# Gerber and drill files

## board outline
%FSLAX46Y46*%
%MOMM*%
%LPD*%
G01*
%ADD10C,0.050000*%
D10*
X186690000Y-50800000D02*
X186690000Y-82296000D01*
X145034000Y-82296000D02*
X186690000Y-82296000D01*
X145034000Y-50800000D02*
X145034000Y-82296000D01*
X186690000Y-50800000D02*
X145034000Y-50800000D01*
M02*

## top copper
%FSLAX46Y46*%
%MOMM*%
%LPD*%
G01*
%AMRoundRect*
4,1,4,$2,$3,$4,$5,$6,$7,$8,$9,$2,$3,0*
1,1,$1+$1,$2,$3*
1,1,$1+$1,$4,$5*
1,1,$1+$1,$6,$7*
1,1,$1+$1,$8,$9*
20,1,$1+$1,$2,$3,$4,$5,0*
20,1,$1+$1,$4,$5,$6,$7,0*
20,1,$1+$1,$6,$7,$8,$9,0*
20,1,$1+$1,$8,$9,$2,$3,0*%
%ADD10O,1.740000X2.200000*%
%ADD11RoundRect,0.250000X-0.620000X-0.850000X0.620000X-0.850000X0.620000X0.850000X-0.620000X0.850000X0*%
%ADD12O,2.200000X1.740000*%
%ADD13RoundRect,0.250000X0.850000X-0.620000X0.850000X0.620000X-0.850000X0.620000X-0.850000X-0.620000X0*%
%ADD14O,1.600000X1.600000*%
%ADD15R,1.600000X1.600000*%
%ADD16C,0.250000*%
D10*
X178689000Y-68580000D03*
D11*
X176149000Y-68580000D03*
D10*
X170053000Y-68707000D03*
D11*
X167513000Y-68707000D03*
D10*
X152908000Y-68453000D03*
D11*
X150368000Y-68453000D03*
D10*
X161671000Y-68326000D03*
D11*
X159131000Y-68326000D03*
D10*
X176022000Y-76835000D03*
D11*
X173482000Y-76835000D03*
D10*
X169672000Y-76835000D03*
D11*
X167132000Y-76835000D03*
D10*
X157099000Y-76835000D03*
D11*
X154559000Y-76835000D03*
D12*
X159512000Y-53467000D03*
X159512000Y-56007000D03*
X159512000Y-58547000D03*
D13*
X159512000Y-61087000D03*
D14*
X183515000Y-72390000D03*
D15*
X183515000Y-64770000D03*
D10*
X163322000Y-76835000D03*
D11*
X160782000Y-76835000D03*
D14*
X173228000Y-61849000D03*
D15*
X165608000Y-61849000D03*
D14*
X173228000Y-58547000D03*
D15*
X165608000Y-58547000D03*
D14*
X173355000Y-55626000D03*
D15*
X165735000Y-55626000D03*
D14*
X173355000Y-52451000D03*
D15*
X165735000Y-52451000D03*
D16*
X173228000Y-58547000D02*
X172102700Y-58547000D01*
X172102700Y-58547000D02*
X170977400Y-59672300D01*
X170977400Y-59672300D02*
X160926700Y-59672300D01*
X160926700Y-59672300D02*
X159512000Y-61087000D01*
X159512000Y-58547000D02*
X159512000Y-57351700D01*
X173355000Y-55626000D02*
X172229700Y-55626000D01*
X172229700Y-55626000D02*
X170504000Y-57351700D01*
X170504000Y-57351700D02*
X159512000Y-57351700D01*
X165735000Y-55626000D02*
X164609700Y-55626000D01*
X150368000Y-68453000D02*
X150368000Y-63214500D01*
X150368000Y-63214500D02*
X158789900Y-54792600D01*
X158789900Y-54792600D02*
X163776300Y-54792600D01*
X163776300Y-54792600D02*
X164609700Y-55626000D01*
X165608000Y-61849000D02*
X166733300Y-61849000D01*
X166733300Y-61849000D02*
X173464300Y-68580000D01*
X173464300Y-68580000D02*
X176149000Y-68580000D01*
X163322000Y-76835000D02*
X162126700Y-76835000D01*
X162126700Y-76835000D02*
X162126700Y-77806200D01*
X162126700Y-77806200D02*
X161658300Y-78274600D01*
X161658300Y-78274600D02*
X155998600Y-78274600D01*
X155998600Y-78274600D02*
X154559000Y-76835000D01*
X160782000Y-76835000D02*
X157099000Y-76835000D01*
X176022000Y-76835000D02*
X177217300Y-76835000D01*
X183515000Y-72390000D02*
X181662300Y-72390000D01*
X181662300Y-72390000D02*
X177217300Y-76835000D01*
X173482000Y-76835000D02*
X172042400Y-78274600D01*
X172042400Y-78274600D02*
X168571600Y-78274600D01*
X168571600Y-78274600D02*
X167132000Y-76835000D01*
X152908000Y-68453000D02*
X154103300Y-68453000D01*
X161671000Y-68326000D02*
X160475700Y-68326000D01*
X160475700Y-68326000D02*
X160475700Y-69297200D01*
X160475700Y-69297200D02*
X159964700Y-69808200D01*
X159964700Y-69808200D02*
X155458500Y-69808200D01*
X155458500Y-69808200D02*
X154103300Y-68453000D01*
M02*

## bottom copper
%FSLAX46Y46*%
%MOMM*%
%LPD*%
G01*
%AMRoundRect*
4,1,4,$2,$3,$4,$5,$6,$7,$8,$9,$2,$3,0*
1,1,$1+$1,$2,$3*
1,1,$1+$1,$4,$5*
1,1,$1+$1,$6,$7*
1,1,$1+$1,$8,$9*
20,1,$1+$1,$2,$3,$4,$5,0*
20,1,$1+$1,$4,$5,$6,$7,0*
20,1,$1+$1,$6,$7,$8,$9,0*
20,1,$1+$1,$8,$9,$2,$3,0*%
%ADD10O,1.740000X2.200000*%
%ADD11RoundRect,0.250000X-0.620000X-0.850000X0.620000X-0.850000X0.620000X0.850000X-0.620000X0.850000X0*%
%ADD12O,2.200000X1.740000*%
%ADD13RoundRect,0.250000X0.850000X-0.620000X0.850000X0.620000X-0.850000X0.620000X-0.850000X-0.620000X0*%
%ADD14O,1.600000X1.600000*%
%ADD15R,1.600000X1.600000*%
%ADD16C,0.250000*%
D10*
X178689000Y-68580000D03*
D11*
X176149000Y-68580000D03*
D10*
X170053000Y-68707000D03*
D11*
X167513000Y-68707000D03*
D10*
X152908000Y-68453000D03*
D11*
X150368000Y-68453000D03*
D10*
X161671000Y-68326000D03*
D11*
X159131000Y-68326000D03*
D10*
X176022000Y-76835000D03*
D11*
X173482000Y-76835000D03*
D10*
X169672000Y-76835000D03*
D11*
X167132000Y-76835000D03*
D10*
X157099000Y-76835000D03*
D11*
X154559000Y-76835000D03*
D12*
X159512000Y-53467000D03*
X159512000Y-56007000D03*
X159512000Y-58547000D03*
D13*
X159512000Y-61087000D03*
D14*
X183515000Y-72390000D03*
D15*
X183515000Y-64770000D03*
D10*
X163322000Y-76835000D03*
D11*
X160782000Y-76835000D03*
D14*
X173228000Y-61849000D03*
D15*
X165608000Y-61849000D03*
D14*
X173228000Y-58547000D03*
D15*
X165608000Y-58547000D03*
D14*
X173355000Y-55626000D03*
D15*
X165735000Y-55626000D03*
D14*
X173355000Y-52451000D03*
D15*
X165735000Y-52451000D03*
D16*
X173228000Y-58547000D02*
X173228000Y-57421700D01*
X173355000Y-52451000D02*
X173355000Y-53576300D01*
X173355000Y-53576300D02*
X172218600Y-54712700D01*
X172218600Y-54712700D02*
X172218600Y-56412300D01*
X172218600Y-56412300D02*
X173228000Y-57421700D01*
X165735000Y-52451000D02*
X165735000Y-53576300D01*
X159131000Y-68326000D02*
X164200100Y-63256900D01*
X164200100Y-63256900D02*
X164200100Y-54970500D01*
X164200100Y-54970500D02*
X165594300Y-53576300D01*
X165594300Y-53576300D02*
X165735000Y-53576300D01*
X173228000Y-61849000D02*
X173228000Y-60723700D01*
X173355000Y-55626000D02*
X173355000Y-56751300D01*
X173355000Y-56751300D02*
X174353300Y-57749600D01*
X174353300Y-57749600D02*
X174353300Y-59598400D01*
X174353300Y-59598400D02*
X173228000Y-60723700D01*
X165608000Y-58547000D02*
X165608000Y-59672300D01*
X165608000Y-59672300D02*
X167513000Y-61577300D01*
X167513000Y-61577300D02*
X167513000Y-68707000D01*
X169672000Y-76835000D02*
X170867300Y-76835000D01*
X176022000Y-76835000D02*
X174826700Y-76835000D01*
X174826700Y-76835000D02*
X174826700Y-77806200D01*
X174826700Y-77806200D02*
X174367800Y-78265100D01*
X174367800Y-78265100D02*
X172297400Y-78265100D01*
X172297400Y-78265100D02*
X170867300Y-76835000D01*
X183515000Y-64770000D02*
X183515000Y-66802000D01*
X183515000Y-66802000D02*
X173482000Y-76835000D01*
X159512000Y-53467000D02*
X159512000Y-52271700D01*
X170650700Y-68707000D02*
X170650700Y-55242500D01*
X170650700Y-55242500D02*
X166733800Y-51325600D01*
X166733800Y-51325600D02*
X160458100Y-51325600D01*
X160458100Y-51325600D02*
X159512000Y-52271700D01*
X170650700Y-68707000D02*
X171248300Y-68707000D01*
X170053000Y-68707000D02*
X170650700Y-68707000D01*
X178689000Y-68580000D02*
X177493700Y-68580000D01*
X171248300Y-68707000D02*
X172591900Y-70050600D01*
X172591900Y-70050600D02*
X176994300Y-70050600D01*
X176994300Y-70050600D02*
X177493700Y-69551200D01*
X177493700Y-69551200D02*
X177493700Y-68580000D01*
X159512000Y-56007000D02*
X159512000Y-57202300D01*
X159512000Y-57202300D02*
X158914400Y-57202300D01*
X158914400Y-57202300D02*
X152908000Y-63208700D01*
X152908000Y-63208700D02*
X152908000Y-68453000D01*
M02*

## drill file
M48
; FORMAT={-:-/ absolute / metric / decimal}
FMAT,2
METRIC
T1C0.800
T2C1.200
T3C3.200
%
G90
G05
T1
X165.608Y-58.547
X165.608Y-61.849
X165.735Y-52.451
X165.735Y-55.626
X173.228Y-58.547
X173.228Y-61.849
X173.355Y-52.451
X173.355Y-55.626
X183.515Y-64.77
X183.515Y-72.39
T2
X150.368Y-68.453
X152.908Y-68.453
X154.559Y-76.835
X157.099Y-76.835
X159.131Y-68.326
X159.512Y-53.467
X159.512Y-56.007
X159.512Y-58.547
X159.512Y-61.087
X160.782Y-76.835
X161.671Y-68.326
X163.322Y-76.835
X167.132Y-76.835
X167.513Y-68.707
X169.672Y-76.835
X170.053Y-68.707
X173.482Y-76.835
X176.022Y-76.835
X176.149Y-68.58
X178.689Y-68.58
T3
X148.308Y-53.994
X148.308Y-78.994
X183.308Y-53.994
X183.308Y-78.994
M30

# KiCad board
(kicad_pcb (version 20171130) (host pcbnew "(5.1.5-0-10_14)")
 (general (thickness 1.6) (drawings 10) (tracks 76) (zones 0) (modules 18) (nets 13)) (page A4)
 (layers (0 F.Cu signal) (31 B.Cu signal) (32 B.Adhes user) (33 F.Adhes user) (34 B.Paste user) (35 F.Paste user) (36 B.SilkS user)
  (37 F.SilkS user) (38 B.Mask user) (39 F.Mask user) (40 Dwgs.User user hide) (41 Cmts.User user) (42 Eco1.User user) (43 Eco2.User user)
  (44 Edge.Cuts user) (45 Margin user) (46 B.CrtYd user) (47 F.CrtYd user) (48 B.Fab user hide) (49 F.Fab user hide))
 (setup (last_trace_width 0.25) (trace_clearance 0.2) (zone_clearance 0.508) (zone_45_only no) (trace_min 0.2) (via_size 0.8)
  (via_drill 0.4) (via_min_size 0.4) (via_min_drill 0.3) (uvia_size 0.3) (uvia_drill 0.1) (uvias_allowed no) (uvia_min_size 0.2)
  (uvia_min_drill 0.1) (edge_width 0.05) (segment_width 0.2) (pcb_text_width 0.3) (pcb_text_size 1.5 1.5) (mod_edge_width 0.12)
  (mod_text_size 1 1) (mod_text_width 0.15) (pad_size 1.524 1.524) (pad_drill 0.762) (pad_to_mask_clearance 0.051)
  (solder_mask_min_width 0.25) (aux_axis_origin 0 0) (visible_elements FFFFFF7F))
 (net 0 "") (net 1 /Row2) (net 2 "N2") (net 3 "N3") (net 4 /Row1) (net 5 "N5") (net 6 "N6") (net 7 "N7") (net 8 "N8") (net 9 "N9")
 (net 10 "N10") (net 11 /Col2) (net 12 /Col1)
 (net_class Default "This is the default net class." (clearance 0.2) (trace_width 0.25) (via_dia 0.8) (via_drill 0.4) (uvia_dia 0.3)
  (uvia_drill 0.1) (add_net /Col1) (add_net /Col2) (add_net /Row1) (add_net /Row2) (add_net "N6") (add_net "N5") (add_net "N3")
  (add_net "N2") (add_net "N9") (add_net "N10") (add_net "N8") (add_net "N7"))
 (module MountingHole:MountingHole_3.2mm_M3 (layer F.Cu) (at 183.308 78.994)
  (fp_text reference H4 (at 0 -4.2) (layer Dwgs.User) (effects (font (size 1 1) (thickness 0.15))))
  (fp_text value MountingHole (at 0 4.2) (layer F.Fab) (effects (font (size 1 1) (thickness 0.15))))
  (pad 1 np_thru_hole circle (at 0 0) (size 3.2 3.2) (drill 3.2) (layers *.Cu *.Mask)))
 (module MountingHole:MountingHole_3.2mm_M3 (layer F.Cu) (at 183.308 53.994)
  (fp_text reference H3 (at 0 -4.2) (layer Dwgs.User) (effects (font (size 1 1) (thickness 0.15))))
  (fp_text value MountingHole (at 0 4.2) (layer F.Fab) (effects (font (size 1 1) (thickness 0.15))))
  (pad 1 np_thru_hole circle (at 0 0) (size 3.2 3.2) (drill 3.2) (layers *.Cu *.Mask)))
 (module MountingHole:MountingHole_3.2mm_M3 (layer F.Cu) (at 148.308 53.994)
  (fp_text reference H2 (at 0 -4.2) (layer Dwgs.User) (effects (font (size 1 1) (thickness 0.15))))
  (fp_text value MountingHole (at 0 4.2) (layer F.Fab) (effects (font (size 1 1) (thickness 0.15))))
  (pad 1 np_thru_hole circle (at 0 0) (size 3.2 3.2) (drill 3.2) (layers *.Cu *.Mask)))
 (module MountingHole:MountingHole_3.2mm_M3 (layer F.Cu) (at 148.308 78.994)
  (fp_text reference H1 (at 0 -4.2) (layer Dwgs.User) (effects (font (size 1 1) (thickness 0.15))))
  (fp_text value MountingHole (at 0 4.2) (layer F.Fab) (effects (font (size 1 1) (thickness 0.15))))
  (pad 1 np_thru_hole circle (at 0 0) (size 3.2 3.2) (drill 3.2) (layers *.Cu *.Mask)))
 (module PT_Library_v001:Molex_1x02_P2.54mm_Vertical (layer F.Cu) (at 176.149 68.58)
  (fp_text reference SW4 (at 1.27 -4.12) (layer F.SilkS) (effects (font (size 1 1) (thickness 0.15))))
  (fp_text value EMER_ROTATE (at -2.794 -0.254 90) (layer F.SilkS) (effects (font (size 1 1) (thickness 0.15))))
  (pad 2 thru_hole oval (at 2.54 0) (size 1.74 2.2) (drill 1.2) (layers *.Cu *.Mask) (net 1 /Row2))
  (pad 1 thru_hole roundrect (at 0 0) (size 1.74 2.2) (drill 1.2) (layers *.Cu *.Mask) (roundrect_rratio 0.143678) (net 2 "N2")))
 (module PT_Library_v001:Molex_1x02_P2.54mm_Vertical (layer F.Cu) (at 167.513 68.707)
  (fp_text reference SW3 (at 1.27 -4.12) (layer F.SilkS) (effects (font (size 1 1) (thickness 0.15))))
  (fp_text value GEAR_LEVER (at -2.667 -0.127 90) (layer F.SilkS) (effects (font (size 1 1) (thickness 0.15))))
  (pad 2 thru_hole oval (at 2.54 0) (size 1.74 2.2) (drill 1.2) (layers *.Cu *.Mask) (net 1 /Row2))
  (pad 1 thru_hole roundrect (at 0 0) (size 1.74 2.2) (drill 1.2) (layers *.Cu *.Mask) (roundrect_rratio 0.143678) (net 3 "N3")))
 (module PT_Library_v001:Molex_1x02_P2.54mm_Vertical (layer F.Cu) (at 150.368 68.453)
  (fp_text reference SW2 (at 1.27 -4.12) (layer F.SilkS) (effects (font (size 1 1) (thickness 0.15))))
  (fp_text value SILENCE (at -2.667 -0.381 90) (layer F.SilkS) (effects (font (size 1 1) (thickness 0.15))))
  (pad 2 thru_hole oval (at 2.54 0) (size 1.74 2.2) (drill 1.2) (layers *.Cu *.Mask) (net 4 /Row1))
  (pad 1 thru_hole roundrect (at 0 0) (size 1.74 2.2) (drill 1.2) (layers *.Cu *.Mask) (roundrect_rratio 0.143678) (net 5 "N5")))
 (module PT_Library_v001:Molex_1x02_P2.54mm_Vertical (layer F.Cu) (at 159.131 68.326)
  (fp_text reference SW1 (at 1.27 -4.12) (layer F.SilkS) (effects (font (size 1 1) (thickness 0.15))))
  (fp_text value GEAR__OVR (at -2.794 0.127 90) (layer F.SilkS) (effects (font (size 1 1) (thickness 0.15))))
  (pad 2 thru_hole oval (at 2.54 0) (size 1.74 2.2) (drill 1.2) (layers *.Cu *.Mask) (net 4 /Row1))
  (pad 1 thru_hole roundrect (at 0 0) (size 1.74 2.2) (drill 1.2) (layers *.Cu *.Mask) (roundrect_rratio 0.143678) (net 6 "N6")))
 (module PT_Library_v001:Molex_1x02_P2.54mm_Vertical (layer F.Cu) (at 173.482 76.835)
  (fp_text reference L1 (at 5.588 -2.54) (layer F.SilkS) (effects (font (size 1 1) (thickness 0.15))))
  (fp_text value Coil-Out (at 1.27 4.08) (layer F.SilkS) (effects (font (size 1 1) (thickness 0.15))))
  (pad 2 thru_hole oval (at 2.54 0) (size 1.74 2.2) (drill 1.2) (layers *.Cu *.Mask) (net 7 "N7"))
  (pad 1 thru_hole roundrect (at 0 0) (size 1.74 2.2) (drill 1.2) (layers *.Cu *.Mask) (roundrect_rratio 0.143678) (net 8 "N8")))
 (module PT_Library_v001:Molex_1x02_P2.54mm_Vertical (layer F.Cu) (at 167.132 76.835)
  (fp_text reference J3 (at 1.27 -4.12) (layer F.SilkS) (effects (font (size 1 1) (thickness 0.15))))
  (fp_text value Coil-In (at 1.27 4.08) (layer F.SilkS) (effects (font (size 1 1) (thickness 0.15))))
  (pad 2 thru_hole oval (at 2.54 0) (size 1.74 2.2) (drill 1.2) (layers *.Cu *.Mask) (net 7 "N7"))
  (pad 1 thru_hole roundrect (at 0 0) (size 1.74 2.2) (drill 1.2) (layers *.Cu *.Mask) (roundrect_rratio 0.143678) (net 8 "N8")))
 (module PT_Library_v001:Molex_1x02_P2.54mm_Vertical (layer F.Cu) (at 154.559 76.835)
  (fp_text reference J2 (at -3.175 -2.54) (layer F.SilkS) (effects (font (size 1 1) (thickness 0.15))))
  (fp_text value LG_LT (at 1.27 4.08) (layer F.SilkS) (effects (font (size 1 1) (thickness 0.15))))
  (pad 2 thru_hole oval (at 2.54 0) (size 1.74 2.2) (drill 1.2) (layers *.Cu *.Mask) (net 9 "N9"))
  (pad 1 thru_hole roundrect (at 0 0) (size 1.74 2.2) (drill 1.2) (layers *.Cu *.Mask) (roundrect_rratio 0.143678) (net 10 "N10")))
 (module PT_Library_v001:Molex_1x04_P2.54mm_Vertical (layer F.Cu) (at 159.512 61.087 90)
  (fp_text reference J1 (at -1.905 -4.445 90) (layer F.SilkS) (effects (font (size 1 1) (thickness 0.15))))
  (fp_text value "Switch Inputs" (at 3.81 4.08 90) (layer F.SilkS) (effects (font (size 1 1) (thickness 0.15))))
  (pad 4 thru_hole oval (at 7.62 0 90) (size 1.74 2.2) (drill 1.2) (layers *.Cu *.Mask) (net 1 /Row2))
  (pad 3 thru_hole oval (at 5.08 0 90) (size 1.74 2.2) (drill 1.2) (layers *.Cu *.Mask) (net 4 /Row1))
  (pad 2 thru_hole oval (at 2.54 0 90) (size 1.74 2.2) (drill 1.2) (layers *.Cu *.Mask) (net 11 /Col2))
  (pad 1 thru_hole roundrect (at 0 0 90) (size 1.74 2.2) (drill 1.2) (layers *.Cu *.Mask) (roundrect_rratio 0.143678) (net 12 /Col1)))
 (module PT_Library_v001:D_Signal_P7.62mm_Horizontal (layer F.Cu) (at 183.515 64.77 270)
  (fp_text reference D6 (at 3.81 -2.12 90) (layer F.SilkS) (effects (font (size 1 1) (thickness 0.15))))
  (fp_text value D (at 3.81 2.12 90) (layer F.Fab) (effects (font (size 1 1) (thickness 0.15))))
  (pad 2 thru_hole oval (at 7.62 0 270) (size 1.6 1.6) (drill 0.8) (layers *.Cu *.Mask) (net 7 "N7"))
  (pad 1 thru_hole rect (at 0 0 270) (size 1.6 1.6) (drill 0.8) (layers *.Cu *.Mask) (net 8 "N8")))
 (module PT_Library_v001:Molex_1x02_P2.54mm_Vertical (layer F.Cu) (at 160.782 76.835)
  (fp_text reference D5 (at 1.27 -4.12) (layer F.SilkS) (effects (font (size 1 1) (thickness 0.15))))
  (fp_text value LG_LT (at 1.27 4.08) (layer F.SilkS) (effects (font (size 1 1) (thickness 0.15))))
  (pad 2 thru_hole oval (at 2.54 0) (size 1.74 2.2) (drill 1.2) (layers *.Cu *.Mask) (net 10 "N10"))
  (pad 1 thru_hole roundrect (at 0 0) (size 1.74 2.2) (drill 1.2) (layers *.Cu *.Mask) (roundrect_rratio 0.143678) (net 9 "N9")))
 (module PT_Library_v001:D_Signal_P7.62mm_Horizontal (layer F.Cu) (at 165.608 61.849)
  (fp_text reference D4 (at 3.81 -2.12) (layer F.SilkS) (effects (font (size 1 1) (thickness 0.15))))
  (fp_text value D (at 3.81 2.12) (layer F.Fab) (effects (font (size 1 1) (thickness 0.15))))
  (pad 2 thru_hole oval (at 7.62 0) (size 1.6 1.6) (drill 0.8) (layers *.Cu *.Mask) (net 11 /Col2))
  (pad 1 thru_hole rect (at 0 0) (size 1.6 1.6) (drill 0.8) (layers *.Cu *.Mask) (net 2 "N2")))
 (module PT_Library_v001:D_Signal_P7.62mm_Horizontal (layer F.Cu) (at 165.608 58.547)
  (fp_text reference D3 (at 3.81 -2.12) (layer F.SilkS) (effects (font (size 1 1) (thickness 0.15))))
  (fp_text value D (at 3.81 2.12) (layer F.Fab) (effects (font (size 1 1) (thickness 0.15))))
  (pad 2 thru_hole oval (at 7.62 0) (size 1.6 1.6) (drill 0.8) (layers *.Cu *.Mask) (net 12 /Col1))
  (pad 1 thru_hole rect (at 0 0) (size 1.6 1.6) (drill 0.8) (layers *.Cu *.Mask) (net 3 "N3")))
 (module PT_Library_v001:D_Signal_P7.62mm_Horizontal (layer F.Cu) (at 165.735 55.626)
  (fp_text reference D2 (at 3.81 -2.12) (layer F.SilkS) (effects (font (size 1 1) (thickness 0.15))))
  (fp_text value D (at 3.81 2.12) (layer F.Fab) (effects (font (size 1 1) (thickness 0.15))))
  (pad 2 thru_hole oval (at 7.62 0) (size 1.6 1.6) (drill 0.8) (layers *.Cu *.Mask) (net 11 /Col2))
  (pad 1 thru_hole rect (at 0 0) (size 1.6 1.6) (drill 0.8) (layers *.Cu *.Mask) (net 5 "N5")))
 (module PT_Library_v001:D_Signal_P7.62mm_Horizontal (layer F.Cu) (at 165.735 52.451)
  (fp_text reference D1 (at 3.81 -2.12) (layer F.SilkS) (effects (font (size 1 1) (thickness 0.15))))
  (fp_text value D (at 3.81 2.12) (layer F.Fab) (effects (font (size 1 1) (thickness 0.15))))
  (pad 2 thru_hole oval (at 7.62 0) (size 1.6 1.6) (drill 0.8) (layers *.Cu *.Mask) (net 12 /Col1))
  (pad 1 thru_hole rect (at 0 0) (size 1.6 1.6) (drill 0.8) (layers *.Cu *.Mask) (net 6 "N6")))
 (gr_line (start 186.69 50.8) (end 186.69 82.296) (layer Edge.Cuts) (width 0.05))
 (gr_line (start 145.034 82.296) (end 186.69 82.296) (layer Edge.Cuts) (width 0.05))
 (gr_line (start 145.034 50.8) (end 145.034 82.296) (layer Edge.Cuts) (width 0.05))
 (gr_line (start 186.69 50.8) (end 145.034 50.8) (layer Edge.Cuts) (width 0.05))
 (segment (start 173.228 58.547) (end 173.228 57.4217) (width 0.25) (layer B.Cu) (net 12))
 (segment (start 173.355 52.451) (end 173.355 53.5763) (width 0.25) (layer B.Cu) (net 12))
 (segment (start 173.355 53.5763) (end 172.2186 54.7127) (width 0.25) (layer B.Cu) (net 12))
 (segment (start 172.2186 54.7127) (end 172.2186 56.4123) (width 0.25) (layer B.Cu) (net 12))
 (segment (start 172.2186 56.4123) (end 173.228 57.4217) (width 0.25) (layer B.Cu) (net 12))
 (segment (start 173.228 58.547) (end 172.1027 58.547) (width 0.25) (layer F.Cu) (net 12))
 (segment (start 172.1027 58.547) (end 170.9774 59.6723) (width 0.25) (layer F.Cu) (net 12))
 (segment (start 170.9774 59.6723) (end 160.9267 59.6723) (width 0.25) (layer F.Cu) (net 12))
 (segment (start 160.9267 59.6723) (end 159.512 61.087) (width 0.25) (layer F.Cu) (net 12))
 (segment (start 165.735 52.451) (end 165.735 53.5763) (width 0.25) (layer B.Cu) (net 6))
 (segment (start 159.131 68.326) (end 164.2001 63.2569) (width 0.25) (layer B.Cu) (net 6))
 (segment (start 164.2001 63.2569) (end 164.2001 54.9705) (width 0.25) (layer B.Cu) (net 6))
 (segment (start 164.2001 54.9705) (end 165.5943 53.5763) (width 0.25) (layer B.Cu) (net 6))
 (segment (start 165.5943 53.5763) (end 165.735 53.5763) (width 0.25) (layer B.Cu) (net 6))
 (segment (start 159.512 58.547) (end 159.512 57.3517) (width 0.25) (layer F.Cu) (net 11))
 (segment (start 173.355 55.626) (end 172.2297 55.626) (width 0.25) (layer F.Cu) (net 11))
 (segment (start 172.2297 55.626) (end 170.504 57.3517) (width 0.25) (layer F.Cu) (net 11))
 (segment (start 170.504 57.3517) (end 159.512 57.3517) (width 0.25) (layer F.Cu) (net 11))
 (segment (start 173.228 61.849) (end 173.228 60.7237) (width 0.25) (layer B.Cu) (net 11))
 (segment (start 173.355 55.626) (end 173.355 56.7513) (width 0.25) (layer B.Cu) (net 11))
 (segment (start 173.355 56.7513) (end 174.3533 57.7496) (width 0.25) (layer B.Cu) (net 11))
 (segment (start 174.3533 57.7496) (end 174.3533 59.5984) (width 0.25) (layer B.Cu) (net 11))
 (segment (start 174.3533 59.5984) (end 173.228 60.7237) (width 0.25) (layer B.Cu) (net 11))
 (segment (start 165.735 55.626) (end 164.6097 55.626) (width 0.25) (layer F.Cu) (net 5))
 (segment (start 150.368 68.453) (end 150.368 63.2145) (width 0.25) (layer F.Cu) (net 5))
 (segment (start 150.368 63.2145) (end 158.7899 54.7926) (width 0.25) (layer F.Cu) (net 5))
 (segment (start 158.7899 54.7926) (end 163.7763 54.7926) (width 0.25) (layer F.Cu) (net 5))
 (segment (start 163.7763 54.7926) (end 164.6097 55.626) (width 0.25) (layer F.Cu) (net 5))
 (segment (start 165.608 58.547) (end 165.608 59.6723) (width 0.25) (layer B.Cu) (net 3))
 (segment (start 165.608 59.6723) (end 167.513 61.5773) (width 0.25) (layer B.Cu) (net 3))
 (segment (start 167.513 61.5773) (end 167.513 68.707) (width 0.25) (layer B.Cu) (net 3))
 (segment (start 165.608 61.849) (end 166.7333 61.849) (width 0.25) (layer F.Cu) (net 2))
 (segment (start 166.7333 61.849) (end 173.4643 68.58) (width 0.25) (layer F.Cu) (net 2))
 (segment (start 173.4643 68.58) (end 176.149 68.58) (width 0.25) (layer F.Cu) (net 2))
 (segment (start 163.322 76.835) (end 162.1267 76.835) (width 0.25) (layer F.Cu) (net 10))
 (segment (start 162.1267 76.835) (end 162.1267 77.8062) (width 0.25) (layer F.Cu) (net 10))
 (segment (start 162.1267 77.8062) (end 161.6583 78.2746) (width 0.25) (layer F.Cu) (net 10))
 (segment (start 161.6583 78.2746) (end 155.9986 78.2746) (width 0.25) (layer F.Cu) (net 10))
 (segment (start 155.9986 78.2746) (end 154.559 76.835) (width 0.25) (layer F.Cu) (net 10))
 (segment (start 160.782 76.835) (end 157.099 76.835) (width 0.25) (layer F.Cu) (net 9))
 (segment (start 169.672 76.835) (end 170.8673 76.835) (width 0.25) (layer B.Cu) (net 7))
 (segment (start 176.022 76.835) (end 174.8267 76.835) (width 0.25) (layer B.Cu) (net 7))
 (segment (start 174.8267 76.835) (end 174.8267 77.8062) (width 0.25) (layer B.Cu) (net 7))
 (segment (start 174.8267 77.8062) (end 174.3678 78.2651) (width 0.25) (layer B.Cu) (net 7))
 (segment (start 174.3678 78.2651) (end 172.2974 78.2651) (width 0.25) (layer B.Cu) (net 7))
 (segment (start 172.2974 78.2651) (end 170.8673 76.835) (width 0.25) (layer B.Cu) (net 7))
 (segment (start 176.022 76.835) (end 177.2173 76.835) (width 0.25) (layer F.Cu) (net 7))
 (segment (start 183.515 72.39) (end 181.6623 72.39) (width 0.25) (layer F.Cu) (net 7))
 (segment (start 181.6623 72.39) (end 177.2173 76.835) (width 0.25) (layer F.Cu) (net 7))
 (segment (start 173.482 76.835) (end 172.0424 78.2746) (width 0.25) (layer F.Cu) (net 8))
 (segment (start 172.0424 78.2746) (end 168.5716 78.2746) (width 0.25) (layer F.Cu) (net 8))
 (segment (start 168.5716 78.2746) (end 167.132 76.835) (width 0.25) (layer F.Cu) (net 8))
 (segment (start 183.515 64.77) (end 183.515 66.802) (width 0.25) (layer B.Cu) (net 8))
 (segment (start 183.515 66.802) (end 173.482 76.835) (width 0.25) (layer B.Cu) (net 8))
 (segment (start 159.512 53.467) (end 159.512 52.2717) (width 0.25) (layer B.Cu) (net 1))
 (segment (start 170.6507 68.707) (end 170.6507 55.2425) (width 0.25) (layer B.Cu) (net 1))
 (segment (start 170.6507 55.2425) (end 166.7338 51.3256) (width 0.25) (layer B.Cu) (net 1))
 (segment (start 166.7338 51.3256) (end 160.4581 51.3256) (width 0.25) (layer B.Cu) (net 1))
 (segment (start 160.4581 51.3256) (end 159.512 52.2717) (width 0.25) (layer B.Cu) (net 1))
 (segment (start 170.6507 68.707) (end 171.2483 68.707) (width 0.25) (layer B.Cu) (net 1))
 (segment (start 170.053 68.707) (end 170.6507 68.707) (width 0.25) (layer B.Cu) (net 1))
 (segment (start 178.689 68.58) (end 177.4937 68.58) (width 0.25) (layer B.Cu) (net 1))
 (segment (start 171.2483 68.707) (end 172.5919 70.0506) (width 0.25) (layer B.Cu) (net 1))
 (segment (start 172.5919 70.0506) (end 176.9943 70.0506) (width 0.25) (layer B.Cu) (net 1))
 (segment (start 176.9943 70.0506) (end 177.4937 69.5512) (width 0.25) (layer B.Cu) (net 1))
 (segment (start 177.4937 69.5512) (end 177.4937 68.58) (width 0.25) (layer B.Cu) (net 1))
 (segment (start 152.908 68.453) (end 154.1033 68.453) (width 0.25) (layer F.Cu) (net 4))
 (segment (start 161.671 68.326) (end 160.4757 68.326) (width 0.25) (layer F.Cu) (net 4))
 (segment (start 160.4757 68.326) (end 160.4757 69.2972) (width 0.25) (layer F.Cu) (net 4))
 (segment (start 160.4757 69.2972) (end 159.9647 69.8082) (width 0.25) (layer F.Cu) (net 4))
 (segment (start 159.9647 69.8082) (end 155.4585 69.8082) (width 0.25) (layer F.Cu) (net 4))
 (segment (start 155.4585 69.8082) (end 154.1033 68.453) (width 0.25) (layer F.Cu) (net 4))
 (segment (start 159.512 56.007) (end 159.512 57.2023) (width 0.25) (layer B.Cu) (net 4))
 (segment (start 159.512 57.2023) (end 158.9144 57.2023) (width 0.25) (layer B.Cu) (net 4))
 (segment (start 158.9144 57.2023) (end 152.908 63.2087) (width 0.25) (layer B.Cu) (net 4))
 (segment (start 152.908 63.2087) (end 152.908 68.453) (width 0.25) (layer B.Cu) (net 4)))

